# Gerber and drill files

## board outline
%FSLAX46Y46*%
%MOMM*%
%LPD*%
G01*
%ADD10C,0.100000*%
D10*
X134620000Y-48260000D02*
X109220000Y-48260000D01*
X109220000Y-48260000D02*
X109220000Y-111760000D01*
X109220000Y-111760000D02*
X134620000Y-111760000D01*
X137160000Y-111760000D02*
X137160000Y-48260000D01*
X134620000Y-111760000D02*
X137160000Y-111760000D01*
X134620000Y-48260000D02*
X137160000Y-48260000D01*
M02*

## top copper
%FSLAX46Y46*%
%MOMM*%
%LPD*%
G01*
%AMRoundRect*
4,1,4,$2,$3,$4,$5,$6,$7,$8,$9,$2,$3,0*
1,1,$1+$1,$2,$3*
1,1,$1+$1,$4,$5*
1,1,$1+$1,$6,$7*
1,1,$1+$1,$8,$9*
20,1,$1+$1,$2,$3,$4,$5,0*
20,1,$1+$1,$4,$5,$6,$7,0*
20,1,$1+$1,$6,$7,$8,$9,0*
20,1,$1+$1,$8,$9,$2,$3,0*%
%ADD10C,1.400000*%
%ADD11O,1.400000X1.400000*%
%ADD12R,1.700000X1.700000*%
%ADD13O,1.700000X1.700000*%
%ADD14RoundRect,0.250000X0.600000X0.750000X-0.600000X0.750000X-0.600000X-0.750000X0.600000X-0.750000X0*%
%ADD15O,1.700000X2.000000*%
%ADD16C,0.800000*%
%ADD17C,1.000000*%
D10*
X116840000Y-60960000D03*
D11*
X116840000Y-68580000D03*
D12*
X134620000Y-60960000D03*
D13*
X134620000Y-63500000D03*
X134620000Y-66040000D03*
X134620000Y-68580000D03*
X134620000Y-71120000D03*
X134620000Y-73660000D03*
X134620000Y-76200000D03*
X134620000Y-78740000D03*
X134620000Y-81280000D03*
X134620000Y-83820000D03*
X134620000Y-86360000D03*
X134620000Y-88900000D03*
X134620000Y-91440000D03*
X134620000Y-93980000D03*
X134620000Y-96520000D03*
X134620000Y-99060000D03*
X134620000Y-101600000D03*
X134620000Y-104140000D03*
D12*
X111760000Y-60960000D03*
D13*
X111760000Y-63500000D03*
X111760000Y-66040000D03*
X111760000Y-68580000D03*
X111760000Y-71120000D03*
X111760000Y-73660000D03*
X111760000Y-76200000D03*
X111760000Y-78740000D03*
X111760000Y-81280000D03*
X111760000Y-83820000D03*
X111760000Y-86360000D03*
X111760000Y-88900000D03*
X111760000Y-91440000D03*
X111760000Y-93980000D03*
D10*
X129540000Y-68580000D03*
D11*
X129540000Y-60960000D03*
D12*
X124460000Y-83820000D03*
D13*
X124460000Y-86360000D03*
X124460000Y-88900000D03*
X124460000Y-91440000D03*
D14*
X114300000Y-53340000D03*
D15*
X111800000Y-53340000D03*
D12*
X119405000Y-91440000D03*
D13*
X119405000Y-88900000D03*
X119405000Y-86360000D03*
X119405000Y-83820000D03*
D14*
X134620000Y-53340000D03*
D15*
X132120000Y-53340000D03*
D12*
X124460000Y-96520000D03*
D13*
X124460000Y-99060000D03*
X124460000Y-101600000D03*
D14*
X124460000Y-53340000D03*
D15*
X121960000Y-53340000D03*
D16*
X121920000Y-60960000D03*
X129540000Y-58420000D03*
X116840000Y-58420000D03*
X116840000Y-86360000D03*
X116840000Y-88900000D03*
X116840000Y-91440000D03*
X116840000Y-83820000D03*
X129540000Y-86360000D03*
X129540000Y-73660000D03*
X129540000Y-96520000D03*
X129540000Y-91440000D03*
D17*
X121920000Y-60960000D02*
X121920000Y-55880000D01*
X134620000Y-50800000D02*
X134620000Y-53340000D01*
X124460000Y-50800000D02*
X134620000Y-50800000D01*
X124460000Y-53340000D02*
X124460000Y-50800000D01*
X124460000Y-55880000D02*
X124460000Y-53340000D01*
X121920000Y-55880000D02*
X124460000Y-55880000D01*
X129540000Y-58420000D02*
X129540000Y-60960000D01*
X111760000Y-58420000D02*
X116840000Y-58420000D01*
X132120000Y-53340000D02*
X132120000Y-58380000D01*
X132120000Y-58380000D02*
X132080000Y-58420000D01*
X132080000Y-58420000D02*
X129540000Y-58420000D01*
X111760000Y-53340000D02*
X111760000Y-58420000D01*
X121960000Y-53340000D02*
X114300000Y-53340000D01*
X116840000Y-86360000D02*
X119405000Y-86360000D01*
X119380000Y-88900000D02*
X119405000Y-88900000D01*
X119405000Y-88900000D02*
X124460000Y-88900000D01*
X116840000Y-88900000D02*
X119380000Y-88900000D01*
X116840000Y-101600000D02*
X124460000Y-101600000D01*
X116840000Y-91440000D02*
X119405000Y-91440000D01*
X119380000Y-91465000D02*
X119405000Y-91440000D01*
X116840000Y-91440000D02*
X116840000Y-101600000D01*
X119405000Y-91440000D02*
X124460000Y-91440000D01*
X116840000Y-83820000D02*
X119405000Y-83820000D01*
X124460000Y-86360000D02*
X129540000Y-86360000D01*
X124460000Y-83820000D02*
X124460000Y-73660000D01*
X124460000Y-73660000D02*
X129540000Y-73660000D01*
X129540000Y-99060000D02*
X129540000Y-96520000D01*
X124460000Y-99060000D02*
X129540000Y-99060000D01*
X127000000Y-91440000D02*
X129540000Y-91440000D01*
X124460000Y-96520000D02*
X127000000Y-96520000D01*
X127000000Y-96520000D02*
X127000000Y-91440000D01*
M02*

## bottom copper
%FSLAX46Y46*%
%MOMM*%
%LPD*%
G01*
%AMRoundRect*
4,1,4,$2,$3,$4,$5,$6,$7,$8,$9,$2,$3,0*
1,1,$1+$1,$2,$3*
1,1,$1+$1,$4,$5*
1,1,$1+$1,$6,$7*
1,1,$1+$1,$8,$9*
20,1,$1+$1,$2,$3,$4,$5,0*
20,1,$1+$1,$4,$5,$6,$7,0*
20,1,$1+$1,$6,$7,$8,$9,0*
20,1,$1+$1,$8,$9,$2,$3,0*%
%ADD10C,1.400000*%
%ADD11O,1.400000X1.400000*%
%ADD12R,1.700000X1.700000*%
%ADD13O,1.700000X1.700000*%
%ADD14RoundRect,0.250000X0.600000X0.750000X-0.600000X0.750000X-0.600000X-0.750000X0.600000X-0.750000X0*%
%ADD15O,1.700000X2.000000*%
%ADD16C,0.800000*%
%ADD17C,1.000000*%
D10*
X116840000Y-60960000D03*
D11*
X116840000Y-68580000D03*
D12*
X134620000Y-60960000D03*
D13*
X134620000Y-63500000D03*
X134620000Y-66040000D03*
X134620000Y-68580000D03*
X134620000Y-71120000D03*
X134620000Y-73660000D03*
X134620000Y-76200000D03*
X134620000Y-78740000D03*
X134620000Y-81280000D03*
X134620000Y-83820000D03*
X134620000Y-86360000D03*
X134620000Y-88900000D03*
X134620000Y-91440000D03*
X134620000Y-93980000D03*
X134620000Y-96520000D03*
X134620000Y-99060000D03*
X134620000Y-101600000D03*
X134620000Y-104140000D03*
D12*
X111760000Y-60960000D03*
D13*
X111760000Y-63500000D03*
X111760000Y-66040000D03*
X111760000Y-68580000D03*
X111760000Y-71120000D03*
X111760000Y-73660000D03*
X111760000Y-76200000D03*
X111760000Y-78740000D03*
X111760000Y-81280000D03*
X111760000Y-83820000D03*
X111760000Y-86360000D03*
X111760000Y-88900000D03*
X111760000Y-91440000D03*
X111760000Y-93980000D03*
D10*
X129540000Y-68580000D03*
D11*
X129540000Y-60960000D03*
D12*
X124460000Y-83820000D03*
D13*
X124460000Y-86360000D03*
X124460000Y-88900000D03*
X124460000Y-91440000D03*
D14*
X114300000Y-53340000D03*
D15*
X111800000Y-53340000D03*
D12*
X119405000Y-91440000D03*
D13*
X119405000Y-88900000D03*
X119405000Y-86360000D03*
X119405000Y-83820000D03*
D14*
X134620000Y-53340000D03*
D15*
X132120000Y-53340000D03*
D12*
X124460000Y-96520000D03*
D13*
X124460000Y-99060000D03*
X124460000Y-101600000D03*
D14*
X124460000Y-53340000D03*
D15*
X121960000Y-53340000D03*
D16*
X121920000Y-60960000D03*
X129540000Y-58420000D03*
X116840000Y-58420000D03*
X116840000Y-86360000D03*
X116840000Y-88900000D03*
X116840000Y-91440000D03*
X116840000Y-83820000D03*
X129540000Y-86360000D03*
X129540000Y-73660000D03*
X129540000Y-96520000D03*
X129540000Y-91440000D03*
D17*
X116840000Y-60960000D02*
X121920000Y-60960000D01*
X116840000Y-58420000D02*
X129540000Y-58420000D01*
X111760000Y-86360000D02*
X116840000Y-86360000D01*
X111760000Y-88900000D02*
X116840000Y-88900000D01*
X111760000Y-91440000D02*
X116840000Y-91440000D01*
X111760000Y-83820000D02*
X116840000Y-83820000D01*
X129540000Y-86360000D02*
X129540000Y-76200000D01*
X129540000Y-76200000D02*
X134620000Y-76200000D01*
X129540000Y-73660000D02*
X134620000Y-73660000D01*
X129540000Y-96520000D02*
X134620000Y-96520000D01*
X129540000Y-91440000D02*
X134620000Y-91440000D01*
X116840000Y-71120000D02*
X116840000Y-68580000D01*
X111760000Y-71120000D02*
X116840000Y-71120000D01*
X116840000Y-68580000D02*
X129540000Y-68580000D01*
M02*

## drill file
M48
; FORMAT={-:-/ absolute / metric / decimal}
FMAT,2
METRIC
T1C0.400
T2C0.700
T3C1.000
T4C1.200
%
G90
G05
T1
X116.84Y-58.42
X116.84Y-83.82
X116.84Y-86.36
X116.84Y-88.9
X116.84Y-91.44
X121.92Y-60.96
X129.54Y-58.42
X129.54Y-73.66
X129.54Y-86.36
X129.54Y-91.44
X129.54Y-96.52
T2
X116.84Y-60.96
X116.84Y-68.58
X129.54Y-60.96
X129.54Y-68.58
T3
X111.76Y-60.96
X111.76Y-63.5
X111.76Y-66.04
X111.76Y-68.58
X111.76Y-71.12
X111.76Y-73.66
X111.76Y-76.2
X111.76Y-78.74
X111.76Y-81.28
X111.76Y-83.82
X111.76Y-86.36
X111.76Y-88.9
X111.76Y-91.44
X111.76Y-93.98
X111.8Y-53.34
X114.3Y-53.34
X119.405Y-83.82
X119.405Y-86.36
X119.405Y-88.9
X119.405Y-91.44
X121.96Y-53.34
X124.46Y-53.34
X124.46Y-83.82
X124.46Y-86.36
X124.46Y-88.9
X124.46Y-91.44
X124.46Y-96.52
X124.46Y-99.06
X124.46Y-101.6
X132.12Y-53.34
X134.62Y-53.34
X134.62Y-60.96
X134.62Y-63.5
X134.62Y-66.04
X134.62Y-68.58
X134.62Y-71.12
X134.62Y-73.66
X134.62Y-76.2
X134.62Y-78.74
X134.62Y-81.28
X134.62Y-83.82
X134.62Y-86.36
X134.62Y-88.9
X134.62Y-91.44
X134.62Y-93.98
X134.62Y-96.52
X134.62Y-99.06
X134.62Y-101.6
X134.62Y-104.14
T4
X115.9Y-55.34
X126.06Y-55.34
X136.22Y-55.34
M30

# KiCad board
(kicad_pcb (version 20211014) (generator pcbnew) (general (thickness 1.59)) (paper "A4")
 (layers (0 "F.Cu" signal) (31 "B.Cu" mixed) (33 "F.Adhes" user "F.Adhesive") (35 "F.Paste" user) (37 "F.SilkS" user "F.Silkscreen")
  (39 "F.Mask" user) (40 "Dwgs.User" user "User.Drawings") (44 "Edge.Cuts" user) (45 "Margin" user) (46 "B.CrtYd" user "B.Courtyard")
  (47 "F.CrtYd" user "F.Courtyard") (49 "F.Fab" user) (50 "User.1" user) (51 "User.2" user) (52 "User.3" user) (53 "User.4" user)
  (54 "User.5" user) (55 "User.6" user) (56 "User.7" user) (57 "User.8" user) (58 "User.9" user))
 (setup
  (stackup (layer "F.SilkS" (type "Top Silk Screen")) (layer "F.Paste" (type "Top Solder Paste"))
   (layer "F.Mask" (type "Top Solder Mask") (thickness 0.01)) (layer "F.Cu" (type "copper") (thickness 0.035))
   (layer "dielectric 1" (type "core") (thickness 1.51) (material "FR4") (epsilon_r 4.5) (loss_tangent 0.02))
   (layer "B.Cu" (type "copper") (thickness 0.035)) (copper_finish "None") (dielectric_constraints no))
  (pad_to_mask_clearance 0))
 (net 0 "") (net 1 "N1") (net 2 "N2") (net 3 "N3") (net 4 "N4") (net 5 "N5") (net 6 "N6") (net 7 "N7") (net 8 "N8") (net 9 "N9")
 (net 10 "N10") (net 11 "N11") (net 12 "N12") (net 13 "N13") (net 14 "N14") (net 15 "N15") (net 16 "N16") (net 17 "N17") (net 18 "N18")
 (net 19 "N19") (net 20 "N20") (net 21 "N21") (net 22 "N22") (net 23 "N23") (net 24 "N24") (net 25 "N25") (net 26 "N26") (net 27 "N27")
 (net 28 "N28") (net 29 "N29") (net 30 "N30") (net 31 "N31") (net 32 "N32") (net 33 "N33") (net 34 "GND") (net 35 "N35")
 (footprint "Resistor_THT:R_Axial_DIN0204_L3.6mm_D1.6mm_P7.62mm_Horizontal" (layer "F.Cu") (at 116.84 60.96 -90)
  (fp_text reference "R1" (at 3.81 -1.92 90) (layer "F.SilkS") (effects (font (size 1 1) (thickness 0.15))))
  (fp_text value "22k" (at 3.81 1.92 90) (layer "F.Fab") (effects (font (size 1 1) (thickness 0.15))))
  (pad "1" thru_hole circle (at 0 0 270) (size 1.4 1.4) (drill 0.7) (layers *.Cu *.Mask) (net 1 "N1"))
  (pad "2" thru_hole oval (at 7.62 0 270) (size 1.4 1.4) (drill 0.7) (layers *.Cu *.Mask) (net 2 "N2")))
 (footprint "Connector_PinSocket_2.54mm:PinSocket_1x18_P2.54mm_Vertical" (layer "F.Cu") (at 134.62 60.96)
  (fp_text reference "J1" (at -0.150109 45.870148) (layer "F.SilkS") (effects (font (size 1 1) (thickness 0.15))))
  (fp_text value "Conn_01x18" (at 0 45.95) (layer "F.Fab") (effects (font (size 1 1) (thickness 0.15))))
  (pad "1" thru_hole rect (at 0 0) (size 1.7 1.7) (drill 1) (layers *.Cu *.Mask) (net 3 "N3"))
  (pad "2" thru_hole oval (at 0 2.54) (size 1.7 1.7) (drill 1) (layers *.Cu *.Mask) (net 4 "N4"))
  (pad "3" thru_hole oval (at 0 5.08) (size 1.7 1.7) (drill 1) (layers *.Cu *.Mask) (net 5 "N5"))
  (pad "4" thru_hole oval (at 0 7.62) (size 1.7 1.7) (drill 1) (layers *.Cu *.Mask) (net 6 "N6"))
  (pad "5" thru_hole oval (at 0 10.16) (size 1.7 1.7) (drill 1) (layers *.Cu *.Mask) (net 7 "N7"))
  (pad "6" thru_hole oval (at 0 12.7) (size 1.7 1.7) (drill 1) (layers *.Cu *.Mask) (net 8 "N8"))
  (pad "7" thru_hole oval (at 0 15.24) (size 1.7 1.7) (drill 1) (layers *.Cu *.Mask) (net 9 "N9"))
  (pad "8" thru_hole oval (at 0 17.78) (size 1.7 1.7) (drill 1) (layers *.Cu *.Mask) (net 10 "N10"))
  (pad "9" thru_hole oval (at 0 20.32) (size 1.7 1.7) (drill 1) (layers *.Cu *.Mask) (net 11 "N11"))
  (pad "10" thru_hole oval (at 0 22.86) (size 1.7 1.7) (drill 1) (layers *.Cu *.Mask) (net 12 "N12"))
  (pad "11" thru_hole oval (at 0 25.4) (size 1.7 1.7) (drill 1) (layers *.Cu *.Mask) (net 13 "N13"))
  (pad "12" thru_hole oval (at 0 27.94) (size 1.7 1.7) (drill 1) (layers *.Cu *.Mask) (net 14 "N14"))
  (pad "13" thru_hole oval (at 0 30.48) (size 1.7 1.7) (drill 1) (layers *.Cu *.Mask) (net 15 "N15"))
  (pad "14" thru_hole oval (at 0 33.02) (size 1.7 1.7) (drill 1) (layers *.Cu *.Mask) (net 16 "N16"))
  (pad "15" thru_hole oval (at 0 35.56) (size 1.7 1.7) (drill 1) (layers *.Cu *.Mask) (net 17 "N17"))
  (pad "16" thru_hole oval (at 0 38.1) (size 1.7 1.7) (drill 1) (layers *.Cu *.Mask) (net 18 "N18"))
  (pad "17" thru_hole oval (at 0 40.64) (size 1.7 1.7) (drill 1) (layers *.Cu *.Mask) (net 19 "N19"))
  (pad "18" thru_hole oval (at 0 43.18) (size 1.7 1.7) (drill 1) (layers *.Cu *.Mask) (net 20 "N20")))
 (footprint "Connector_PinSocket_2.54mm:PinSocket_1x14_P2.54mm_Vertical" (layer "F.Cu") (at 111.76 60.96)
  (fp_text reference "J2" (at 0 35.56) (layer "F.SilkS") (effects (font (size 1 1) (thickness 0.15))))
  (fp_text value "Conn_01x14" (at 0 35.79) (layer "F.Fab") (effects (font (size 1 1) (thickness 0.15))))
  (pad "1" thru_hole rect (at 0 0) (size 1.7 1.7) (drill 1) (layers *.Cu *.Mask) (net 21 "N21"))
  (pad "2" thru_hole oval (at 0 2.54) (size 1.7 1.7) (drill 1) (layers *.Cu *.Mask) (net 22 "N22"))
  (pad "3" thru_hole oval (at 0 5.08) (size 1.7 1.7) (drill 1) (layers *.Cu *.Mask) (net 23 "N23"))
  (pad "4" thru_hole oval (at 0 7.62) (size 1.7 1.7) (drill 1) (layers *.Cu *.Mask) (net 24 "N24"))
  (pad "5" thru_hole oval (at 0 10.16) (size 1.7 1.7) (drill 1) (layers *.Cu *.Mask) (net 2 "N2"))
  (pad "6" thru_hole oval (at 0 12.7) (size 1.7 1.7) (drill 1) (layers *.Cu *.Mask) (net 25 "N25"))
  (pad "7" thru_hole oval (at 0 15.24) (size 1.7 1.7) (drill 1) (layers *.Cu *.Mask) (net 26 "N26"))
  (pad "8" thru_hole oval (at 0 17.78) (size 1.7 1.7) (drill 1) (layers *.Cu *.Mask) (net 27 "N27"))
  (pad "9" thru_hole oval (at 0 20.32) (size 1.7 1.7) (drill 1) (layers *.Cu *.Mask) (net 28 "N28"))
  (pad "10" thru_hole oval (at 0 22.86) (size 1.7 1.7) (drill 1) (layers *.Cu *.Mask) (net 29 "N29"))
  (pad "11" thru_hole oval (at 0 25.4) (size 1.7 1.7) (drill 1) (layers *.Cu *.Mask) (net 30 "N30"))
  (pad "12" thru_hole oval (at 0 27.94) (size 1.7 1.7) (drill 1) (layers *.Cu *.Mask) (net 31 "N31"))
  (pad "13" thru_hole oval (at 0 30.48) (size 1.7 1.7) (drill 1) (layers *.Cu *.Mask) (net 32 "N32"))
  (pad "14" thru_hole oval (at 0 33.02) (size 1.7 1.7) (drill 1) (layers *.Cu *.Mask) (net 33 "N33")))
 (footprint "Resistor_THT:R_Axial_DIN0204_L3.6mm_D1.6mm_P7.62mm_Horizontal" (layer "F.Cu") (at 129.54 68.58 90)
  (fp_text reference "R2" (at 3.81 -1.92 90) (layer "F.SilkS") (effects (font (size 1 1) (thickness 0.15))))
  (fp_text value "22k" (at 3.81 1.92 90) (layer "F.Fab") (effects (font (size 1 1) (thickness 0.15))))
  (pad "1" thru_hole circle (at 0 0 90) (size 1.4 1.4) (drill 0.7) (layers *.Cu *.Mask) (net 2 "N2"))
  (pad "2" thru_hole oval (at 7.62 0 90) (size 1.4 1.4) (drill 0.7) (layers *.Cu *.Mask) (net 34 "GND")))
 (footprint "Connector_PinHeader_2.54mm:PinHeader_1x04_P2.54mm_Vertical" (layer "B.Cu") (at 124.46 83.82 180)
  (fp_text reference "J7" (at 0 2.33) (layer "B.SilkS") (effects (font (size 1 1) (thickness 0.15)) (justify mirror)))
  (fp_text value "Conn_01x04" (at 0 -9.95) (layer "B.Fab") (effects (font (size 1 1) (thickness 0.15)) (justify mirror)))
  (pad "1" thru_hole rect (at 0 0 180) (size 1.7 1.7) (drill 1) (layers *.Cu *.Mask) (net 8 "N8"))
  (pad "2" thru_hole oval (at 0 -2.54 180) (size 1.7 1.7) (drill 1) (layers *.Cu *.Mask) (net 9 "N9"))
  (pad "3" thru_hole oval (at 0 -5.08 180) (size 1.7 1.7) (drill 1) (layers *.Cu *.Mask) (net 31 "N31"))
  (pad "4" thru_hole oval (at 0 -7.62 180) (size 1.7 1.7) (drill 1) (layers *.Cu *.Mask) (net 32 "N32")))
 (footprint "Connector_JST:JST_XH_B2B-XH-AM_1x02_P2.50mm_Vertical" (layer "B.Cu") (at 114.3 53.34 180)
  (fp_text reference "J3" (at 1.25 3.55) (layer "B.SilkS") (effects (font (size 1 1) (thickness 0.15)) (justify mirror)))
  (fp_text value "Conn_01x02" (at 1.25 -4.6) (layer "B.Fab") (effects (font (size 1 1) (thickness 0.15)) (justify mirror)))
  (pad "" np_thru_hole circle (at -1.6 -2 180) (size 1.2 1.2) (drill 1.2) (layers *.Cu *.Mask))
  (pad "1" thru_hole roundrect (at 0 0 180) (size 1.7 2) (drill 1) (layers *.Cu *.Mask) (roundrect_rratio 0.147059) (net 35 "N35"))
  (pad "2" thru_hole oval (at 2.5 0 180) (size 1.7 2) (drill 1) (layers *.Cu *.Mask) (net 34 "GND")))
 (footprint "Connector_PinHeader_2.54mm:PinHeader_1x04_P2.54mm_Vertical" (layer "B.Cu") (at 119.405 91.44)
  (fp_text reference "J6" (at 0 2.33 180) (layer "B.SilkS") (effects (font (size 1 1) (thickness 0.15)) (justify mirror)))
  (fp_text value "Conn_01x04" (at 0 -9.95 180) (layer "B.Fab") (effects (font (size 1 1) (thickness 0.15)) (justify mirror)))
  (pad "1" thru_hole rect (at 0 0) (size 1.7 1.7) (drill 1) (layers *.Cu *.Mask) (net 32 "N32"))
  (pad "2" thru_hole oval (at 0 -2.54) (size 1.7 1.7) (drill 1) (layers *.Cu *.Mask) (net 31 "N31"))
  (pad "3" thru_hole oval (at 0 -5.08) (size 1.7 1.7) (drill 1) (layers *.Cu *.Mask) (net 30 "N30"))
  (pad "4" thru_hole oval (at 0 -7.62) (size 1.7 1.7) (drill 1) (layers *.Cu *.Mask) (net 29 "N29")))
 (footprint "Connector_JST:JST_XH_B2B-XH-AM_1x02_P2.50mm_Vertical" (layer "B.Cu") (at 134.62 53.34 180)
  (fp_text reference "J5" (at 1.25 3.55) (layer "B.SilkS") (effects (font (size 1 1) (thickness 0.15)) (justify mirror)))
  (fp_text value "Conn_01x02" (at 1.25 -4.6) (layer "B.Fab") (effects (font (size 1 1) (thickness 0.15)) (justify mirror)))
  (pad "" np_thru_hole circle (at -1.6 -2 180) (size 1.2 1.2) (drill 1.2) (layers *.Cu *.Mask))
  (pad "1" thru_hole roundrect (at 0 0 180) (size 1.7 2) (drill 1) (layers *.Cu *.Mask) (roundrect_rratio 0.147059) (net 1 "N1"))
  (pad "2" thru_hole oval (at 2.5 0 180) (size 1.7 2) (drill 1) (layers *.Cu *.Mask) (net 34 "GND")))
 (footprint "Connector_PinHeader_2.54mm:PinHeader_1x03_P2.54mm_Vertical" (layer "B.Cu") (at 124.46 96.52 180)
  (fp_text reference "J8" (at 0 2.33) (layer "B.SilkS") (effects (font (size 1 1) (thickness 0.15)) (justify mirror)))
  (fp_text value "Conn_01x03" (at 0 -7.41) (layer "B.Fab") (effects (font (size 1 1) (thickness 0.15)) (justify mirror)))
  (pad "1" thru_hole rect (at 0 0 180) (size 1.7 1.7) (drill 1) (layers *.Cu *.Mask) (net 15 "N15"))
  (pad "2" thru_hole oval (at 0 -2.54 180) (size 1.7 1.7) (drill 1) (layers *.Cu *.Mask) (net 17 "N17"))
  (pad "3" thru_hole oval (at 0 -5.08 180) (size 1.7 1.7) (drill 1) (layers *.Cu *.Mask) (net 32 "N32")))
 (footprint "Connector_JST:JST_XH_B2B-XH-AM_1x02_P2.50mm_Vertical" (layer "B.Cu") (at 124.46 53.34 180)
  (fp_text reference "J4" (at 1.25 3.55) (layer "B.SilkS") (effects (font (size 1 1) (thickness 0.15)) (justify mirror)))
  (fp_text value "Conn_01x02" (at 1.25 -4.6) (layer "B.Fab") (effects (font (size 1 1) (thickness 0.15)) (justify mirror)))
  (pad "" np_thru_hole circle (at -1.6 -2 180) (size 1.2 1.2) (drill 1.2) (layers *.Cu *.Mask))
  (pad "1" thru_hole roundrect (at 0 0 180) (size 1.7 2) (drill 1) (layers *.Cu *.Mask) (roundrect_rratio 0.147059) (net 1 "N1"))
  (pad "2" thru_hole oval (at 2.5 0 180) (size 1.7 2) (drill 1) (layers *.Cu *.Mask) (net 35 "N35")))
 (gr_line (start 134.62 48.26) (end 109.22 48.26) (layer "Edge.Cuts") (width 0.1))
 (gr_line (start 109.22 48.26) (end 109.22 111.76) (layer "Edge.Cuts") (width 0.1))
 (gr_line (start 109.22 111.76) (end 134.62 111.76) (layer "Edge.Cuts") (width 0.1))
 (gr_line (start 137.16 111.76) (end 137.16 48.26) (layer "Edge.Cuts") (width 0.1))
 (gr_line (start 134.62 111.76) (end 137.16 111.76) (layer "Edge.Cuts") (width 0.1))
 (gr_line (start 134.62 48.26) (end 137.16 48.26) (layer "Edge.Cuts") (width 0.1))
 (segment (start 121.92 60.96) (end 121.92 55.88) (width 1) (layer "F.Cu") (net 1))
 (segment (start 134.62 50.8) (end 134.62 53.34) (width 1) (layer "F.Cu") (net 1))
 (segment (start 124.46 50.8) (end 134.62 50.8) (width 1) (layer "F.Cu") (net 1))
 (segment (start 124.46 53.34) (end 124.46 50.8) (width 1) (layer "F.Cu") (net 1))
 (segment (start 124.46 55.88) (end 124.46 53.34) (width 1) (layer "F.Cu") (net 1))
 (segment (start 121.92 55.88) (end 124.46 55.88) (width 1) (layer "F.Cu") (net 1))
 (via (at 121.92 60.96) (size 0.8) (drill 0.4) (layers "F.Cu" "B.Cu") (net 1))
 (segment (start 116.84 60.96) (end 121.92 60.96) (width 1) (layer "B.Cu") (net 1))
 (segment (start 129.54 58.42) (end 129.54 60.96) (width 1) (layer "F.Cu") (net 34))
 (segment (start 111.76 58.42) (end 116.84 58.42) (width 1) (layer "F.Cu") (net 34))
 (segment (start 132.12 53.34) (end 132.12 58.38) (width 1) (layer "F.Cu") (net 34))
 (segment (start 132.12 58.38) (end 132.08 58.42) (width 1) (layer "F.Cu") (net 34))
 (segment (start 132.08 58.42) (end 129.54 58.42) (width 1) (layer "F.Cu") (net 34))
 (segment (start 111.76 53.34) (end 111.76 58.42) (width 1) (layer "F.Cu") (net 34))
 (via (at 129.54 58.42) (size 0.8) (drill 0.4) (layers "F.Cu" "B.Cu") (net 34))
 (via (at 116.84 58.42) (size 0.8) (drill 0.4) (layers "F.Cu" "B.Cu") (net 34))
 (segment (start 116.84 58.42) (end 129.54 58.42) (width 1) (layer "B.Cu") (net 34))
 (segment (start 121.96 53.34) (end 114.3 53.34) (width 1) (layer "F.Cu") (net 35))
 (segment (start 116.84 86.36) (end 119.405 86.36) (width 1) (layer "F.Cu") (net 30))
 (via (at 116.84 86.36) (size 0.8) (drill 0.4) (layers "F.Cu" "B.Cu") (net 30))
 (segment (start 111.76 86.36) (end 116.84 86.36) (width 1) (layer "B.Cu") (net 30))
 (segment (start 119.38 88.9) (end 119.405 88.9) (width 1) (layer "F.Cu") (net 31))
 (segment (start 119.405 88.9) (end 124.46 88.9) (width 1) (layer "F.Cu") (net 31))
 (segment (start 116.84 88.9) (end 119.38 88.9) (width 1) (layer "F.Cu") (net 31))
 (via (at 116.84 88.9) (size 0.8) (drill 0.4) (layers "F.Cu" "B.Cu") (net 31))
 (segment (start 111.76 88.9) (end 116.84 88.9) (width 1) (layer "B.Cu") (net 31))
 (segment (start 116.84 101.6) (end 124.46 101.6) (width 1) (layer "F.Cu") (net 32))
 (segment (start 116.84 91.44) (end 119.405 91.44) (width 1) (layer "F.Cu") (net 32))
 (segment (start 119.38 91.465) (end 119.405 91.44) (width 1) (layer "F.Cu") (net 32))
 (segment (start 116.84 91.44) (end 116.84 101.6) (width 1) (layer "F.Cu") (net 32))
 (segment (start 119.405 91.44) (end 124.46 91.44) (width 1) (layer "F.Cu") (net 32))
 (via (at 116.84 91.44) (size 0.8) (drill 0.4) (layers "F.Cu" "B.Cu") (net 32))
 (segment (start 111.76 91.44) (end 116.84 91.44) (width 1) (layer "B.Cu") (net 32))
 (segment (start 116.84 83.82) (end 119.405 83.82) (width 1) (layer "F.Cu") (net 29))
 (via (at 116.84 83.82) (size 0.8) (drill 0.4) (layers "F.Cu" "B.Cu") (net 29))
 (segment (start 111.76 83.82) (end 116.84 83.82) (width 1) (layer "B.Cu") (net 29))
 (segment (start 124.46 86.36) (end 129.54 86.36) (width 1) (layer "F.Cu") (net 9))
 (via (at 129.54 86.36) (size 0.8) (drill 0.4) (layers "F.Cu" "B.Cu") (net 9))
 (segment (start 129.54 86.36) (end 129.54 76.2) (width 1) (layer "B.Cu") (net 9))
 (segment (start 129.54 76.2) (end 134.62 76.2) (width 1) (layer "B.Cu") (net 9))
 (segment (start 124.46 83.82) (end 124.46 73.66) (width 1) (layer "F.Cu") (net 8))
 (segment (start 124.46 73.66) (end 129.54 73.66) (width 1) (layer "F.Cu") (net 8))
 (via (at 129.54 73.66) (size 0.8) (drill 0.4) (layers "F.Cu" "B.Cu") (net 8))
 (segment (start 129.54 73.66) (end 134.62 73.66) (width 1) (layer "B.Cu") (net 8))
 (segment (start 129.54 99.06) (end 129.54 96.52) (width 1) (layer "F.Cu") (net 17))
 (segment (start 124.46 99.06) (end 129.54 99.06) (width 1) (layer "F.Cu") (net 17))
 (via (at 129.54 96.52) (size 0.8) (drill 0.4) (layers "F.Cu" "B.Cu") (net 17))
 (segment (start 129.54 96.52) (end 134.62 96.52) (width 1) (layer "B.Cu") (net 17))
 (segment (start 127 91.44) (end 129.54 91.44) (width 1) (layer "F.Cu") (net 15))
 (segment (start 124.46 96.52) (end 127 96.52) (width 1) (layer "F.Cu") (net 15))
 (segment (start 127 96.52) (end 127 91.44) (width 1) (layer "F.Cu") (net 15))
 (via (at 129.54 91.44) (size 0.8) (drill 0.4) (layers "F.Cu" "B.Cu") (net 15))
 (segment (start 129.54 91.44) (end 134.62 91.44) (width 1) (layer "B.Cu") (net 15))
 (segment (start 116.84 71.12) (end 116.84 68.58) (width 1) (layer "B.Cu") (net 2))
 (segment (start 111.76 71.12) (end 116.84 71.12) (width 1) (layer "B.Cu") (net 2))
 (segment (start 116.84 68.58) (end 129.54 68.58) (width 1) (layer "B.Cu") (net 2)))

